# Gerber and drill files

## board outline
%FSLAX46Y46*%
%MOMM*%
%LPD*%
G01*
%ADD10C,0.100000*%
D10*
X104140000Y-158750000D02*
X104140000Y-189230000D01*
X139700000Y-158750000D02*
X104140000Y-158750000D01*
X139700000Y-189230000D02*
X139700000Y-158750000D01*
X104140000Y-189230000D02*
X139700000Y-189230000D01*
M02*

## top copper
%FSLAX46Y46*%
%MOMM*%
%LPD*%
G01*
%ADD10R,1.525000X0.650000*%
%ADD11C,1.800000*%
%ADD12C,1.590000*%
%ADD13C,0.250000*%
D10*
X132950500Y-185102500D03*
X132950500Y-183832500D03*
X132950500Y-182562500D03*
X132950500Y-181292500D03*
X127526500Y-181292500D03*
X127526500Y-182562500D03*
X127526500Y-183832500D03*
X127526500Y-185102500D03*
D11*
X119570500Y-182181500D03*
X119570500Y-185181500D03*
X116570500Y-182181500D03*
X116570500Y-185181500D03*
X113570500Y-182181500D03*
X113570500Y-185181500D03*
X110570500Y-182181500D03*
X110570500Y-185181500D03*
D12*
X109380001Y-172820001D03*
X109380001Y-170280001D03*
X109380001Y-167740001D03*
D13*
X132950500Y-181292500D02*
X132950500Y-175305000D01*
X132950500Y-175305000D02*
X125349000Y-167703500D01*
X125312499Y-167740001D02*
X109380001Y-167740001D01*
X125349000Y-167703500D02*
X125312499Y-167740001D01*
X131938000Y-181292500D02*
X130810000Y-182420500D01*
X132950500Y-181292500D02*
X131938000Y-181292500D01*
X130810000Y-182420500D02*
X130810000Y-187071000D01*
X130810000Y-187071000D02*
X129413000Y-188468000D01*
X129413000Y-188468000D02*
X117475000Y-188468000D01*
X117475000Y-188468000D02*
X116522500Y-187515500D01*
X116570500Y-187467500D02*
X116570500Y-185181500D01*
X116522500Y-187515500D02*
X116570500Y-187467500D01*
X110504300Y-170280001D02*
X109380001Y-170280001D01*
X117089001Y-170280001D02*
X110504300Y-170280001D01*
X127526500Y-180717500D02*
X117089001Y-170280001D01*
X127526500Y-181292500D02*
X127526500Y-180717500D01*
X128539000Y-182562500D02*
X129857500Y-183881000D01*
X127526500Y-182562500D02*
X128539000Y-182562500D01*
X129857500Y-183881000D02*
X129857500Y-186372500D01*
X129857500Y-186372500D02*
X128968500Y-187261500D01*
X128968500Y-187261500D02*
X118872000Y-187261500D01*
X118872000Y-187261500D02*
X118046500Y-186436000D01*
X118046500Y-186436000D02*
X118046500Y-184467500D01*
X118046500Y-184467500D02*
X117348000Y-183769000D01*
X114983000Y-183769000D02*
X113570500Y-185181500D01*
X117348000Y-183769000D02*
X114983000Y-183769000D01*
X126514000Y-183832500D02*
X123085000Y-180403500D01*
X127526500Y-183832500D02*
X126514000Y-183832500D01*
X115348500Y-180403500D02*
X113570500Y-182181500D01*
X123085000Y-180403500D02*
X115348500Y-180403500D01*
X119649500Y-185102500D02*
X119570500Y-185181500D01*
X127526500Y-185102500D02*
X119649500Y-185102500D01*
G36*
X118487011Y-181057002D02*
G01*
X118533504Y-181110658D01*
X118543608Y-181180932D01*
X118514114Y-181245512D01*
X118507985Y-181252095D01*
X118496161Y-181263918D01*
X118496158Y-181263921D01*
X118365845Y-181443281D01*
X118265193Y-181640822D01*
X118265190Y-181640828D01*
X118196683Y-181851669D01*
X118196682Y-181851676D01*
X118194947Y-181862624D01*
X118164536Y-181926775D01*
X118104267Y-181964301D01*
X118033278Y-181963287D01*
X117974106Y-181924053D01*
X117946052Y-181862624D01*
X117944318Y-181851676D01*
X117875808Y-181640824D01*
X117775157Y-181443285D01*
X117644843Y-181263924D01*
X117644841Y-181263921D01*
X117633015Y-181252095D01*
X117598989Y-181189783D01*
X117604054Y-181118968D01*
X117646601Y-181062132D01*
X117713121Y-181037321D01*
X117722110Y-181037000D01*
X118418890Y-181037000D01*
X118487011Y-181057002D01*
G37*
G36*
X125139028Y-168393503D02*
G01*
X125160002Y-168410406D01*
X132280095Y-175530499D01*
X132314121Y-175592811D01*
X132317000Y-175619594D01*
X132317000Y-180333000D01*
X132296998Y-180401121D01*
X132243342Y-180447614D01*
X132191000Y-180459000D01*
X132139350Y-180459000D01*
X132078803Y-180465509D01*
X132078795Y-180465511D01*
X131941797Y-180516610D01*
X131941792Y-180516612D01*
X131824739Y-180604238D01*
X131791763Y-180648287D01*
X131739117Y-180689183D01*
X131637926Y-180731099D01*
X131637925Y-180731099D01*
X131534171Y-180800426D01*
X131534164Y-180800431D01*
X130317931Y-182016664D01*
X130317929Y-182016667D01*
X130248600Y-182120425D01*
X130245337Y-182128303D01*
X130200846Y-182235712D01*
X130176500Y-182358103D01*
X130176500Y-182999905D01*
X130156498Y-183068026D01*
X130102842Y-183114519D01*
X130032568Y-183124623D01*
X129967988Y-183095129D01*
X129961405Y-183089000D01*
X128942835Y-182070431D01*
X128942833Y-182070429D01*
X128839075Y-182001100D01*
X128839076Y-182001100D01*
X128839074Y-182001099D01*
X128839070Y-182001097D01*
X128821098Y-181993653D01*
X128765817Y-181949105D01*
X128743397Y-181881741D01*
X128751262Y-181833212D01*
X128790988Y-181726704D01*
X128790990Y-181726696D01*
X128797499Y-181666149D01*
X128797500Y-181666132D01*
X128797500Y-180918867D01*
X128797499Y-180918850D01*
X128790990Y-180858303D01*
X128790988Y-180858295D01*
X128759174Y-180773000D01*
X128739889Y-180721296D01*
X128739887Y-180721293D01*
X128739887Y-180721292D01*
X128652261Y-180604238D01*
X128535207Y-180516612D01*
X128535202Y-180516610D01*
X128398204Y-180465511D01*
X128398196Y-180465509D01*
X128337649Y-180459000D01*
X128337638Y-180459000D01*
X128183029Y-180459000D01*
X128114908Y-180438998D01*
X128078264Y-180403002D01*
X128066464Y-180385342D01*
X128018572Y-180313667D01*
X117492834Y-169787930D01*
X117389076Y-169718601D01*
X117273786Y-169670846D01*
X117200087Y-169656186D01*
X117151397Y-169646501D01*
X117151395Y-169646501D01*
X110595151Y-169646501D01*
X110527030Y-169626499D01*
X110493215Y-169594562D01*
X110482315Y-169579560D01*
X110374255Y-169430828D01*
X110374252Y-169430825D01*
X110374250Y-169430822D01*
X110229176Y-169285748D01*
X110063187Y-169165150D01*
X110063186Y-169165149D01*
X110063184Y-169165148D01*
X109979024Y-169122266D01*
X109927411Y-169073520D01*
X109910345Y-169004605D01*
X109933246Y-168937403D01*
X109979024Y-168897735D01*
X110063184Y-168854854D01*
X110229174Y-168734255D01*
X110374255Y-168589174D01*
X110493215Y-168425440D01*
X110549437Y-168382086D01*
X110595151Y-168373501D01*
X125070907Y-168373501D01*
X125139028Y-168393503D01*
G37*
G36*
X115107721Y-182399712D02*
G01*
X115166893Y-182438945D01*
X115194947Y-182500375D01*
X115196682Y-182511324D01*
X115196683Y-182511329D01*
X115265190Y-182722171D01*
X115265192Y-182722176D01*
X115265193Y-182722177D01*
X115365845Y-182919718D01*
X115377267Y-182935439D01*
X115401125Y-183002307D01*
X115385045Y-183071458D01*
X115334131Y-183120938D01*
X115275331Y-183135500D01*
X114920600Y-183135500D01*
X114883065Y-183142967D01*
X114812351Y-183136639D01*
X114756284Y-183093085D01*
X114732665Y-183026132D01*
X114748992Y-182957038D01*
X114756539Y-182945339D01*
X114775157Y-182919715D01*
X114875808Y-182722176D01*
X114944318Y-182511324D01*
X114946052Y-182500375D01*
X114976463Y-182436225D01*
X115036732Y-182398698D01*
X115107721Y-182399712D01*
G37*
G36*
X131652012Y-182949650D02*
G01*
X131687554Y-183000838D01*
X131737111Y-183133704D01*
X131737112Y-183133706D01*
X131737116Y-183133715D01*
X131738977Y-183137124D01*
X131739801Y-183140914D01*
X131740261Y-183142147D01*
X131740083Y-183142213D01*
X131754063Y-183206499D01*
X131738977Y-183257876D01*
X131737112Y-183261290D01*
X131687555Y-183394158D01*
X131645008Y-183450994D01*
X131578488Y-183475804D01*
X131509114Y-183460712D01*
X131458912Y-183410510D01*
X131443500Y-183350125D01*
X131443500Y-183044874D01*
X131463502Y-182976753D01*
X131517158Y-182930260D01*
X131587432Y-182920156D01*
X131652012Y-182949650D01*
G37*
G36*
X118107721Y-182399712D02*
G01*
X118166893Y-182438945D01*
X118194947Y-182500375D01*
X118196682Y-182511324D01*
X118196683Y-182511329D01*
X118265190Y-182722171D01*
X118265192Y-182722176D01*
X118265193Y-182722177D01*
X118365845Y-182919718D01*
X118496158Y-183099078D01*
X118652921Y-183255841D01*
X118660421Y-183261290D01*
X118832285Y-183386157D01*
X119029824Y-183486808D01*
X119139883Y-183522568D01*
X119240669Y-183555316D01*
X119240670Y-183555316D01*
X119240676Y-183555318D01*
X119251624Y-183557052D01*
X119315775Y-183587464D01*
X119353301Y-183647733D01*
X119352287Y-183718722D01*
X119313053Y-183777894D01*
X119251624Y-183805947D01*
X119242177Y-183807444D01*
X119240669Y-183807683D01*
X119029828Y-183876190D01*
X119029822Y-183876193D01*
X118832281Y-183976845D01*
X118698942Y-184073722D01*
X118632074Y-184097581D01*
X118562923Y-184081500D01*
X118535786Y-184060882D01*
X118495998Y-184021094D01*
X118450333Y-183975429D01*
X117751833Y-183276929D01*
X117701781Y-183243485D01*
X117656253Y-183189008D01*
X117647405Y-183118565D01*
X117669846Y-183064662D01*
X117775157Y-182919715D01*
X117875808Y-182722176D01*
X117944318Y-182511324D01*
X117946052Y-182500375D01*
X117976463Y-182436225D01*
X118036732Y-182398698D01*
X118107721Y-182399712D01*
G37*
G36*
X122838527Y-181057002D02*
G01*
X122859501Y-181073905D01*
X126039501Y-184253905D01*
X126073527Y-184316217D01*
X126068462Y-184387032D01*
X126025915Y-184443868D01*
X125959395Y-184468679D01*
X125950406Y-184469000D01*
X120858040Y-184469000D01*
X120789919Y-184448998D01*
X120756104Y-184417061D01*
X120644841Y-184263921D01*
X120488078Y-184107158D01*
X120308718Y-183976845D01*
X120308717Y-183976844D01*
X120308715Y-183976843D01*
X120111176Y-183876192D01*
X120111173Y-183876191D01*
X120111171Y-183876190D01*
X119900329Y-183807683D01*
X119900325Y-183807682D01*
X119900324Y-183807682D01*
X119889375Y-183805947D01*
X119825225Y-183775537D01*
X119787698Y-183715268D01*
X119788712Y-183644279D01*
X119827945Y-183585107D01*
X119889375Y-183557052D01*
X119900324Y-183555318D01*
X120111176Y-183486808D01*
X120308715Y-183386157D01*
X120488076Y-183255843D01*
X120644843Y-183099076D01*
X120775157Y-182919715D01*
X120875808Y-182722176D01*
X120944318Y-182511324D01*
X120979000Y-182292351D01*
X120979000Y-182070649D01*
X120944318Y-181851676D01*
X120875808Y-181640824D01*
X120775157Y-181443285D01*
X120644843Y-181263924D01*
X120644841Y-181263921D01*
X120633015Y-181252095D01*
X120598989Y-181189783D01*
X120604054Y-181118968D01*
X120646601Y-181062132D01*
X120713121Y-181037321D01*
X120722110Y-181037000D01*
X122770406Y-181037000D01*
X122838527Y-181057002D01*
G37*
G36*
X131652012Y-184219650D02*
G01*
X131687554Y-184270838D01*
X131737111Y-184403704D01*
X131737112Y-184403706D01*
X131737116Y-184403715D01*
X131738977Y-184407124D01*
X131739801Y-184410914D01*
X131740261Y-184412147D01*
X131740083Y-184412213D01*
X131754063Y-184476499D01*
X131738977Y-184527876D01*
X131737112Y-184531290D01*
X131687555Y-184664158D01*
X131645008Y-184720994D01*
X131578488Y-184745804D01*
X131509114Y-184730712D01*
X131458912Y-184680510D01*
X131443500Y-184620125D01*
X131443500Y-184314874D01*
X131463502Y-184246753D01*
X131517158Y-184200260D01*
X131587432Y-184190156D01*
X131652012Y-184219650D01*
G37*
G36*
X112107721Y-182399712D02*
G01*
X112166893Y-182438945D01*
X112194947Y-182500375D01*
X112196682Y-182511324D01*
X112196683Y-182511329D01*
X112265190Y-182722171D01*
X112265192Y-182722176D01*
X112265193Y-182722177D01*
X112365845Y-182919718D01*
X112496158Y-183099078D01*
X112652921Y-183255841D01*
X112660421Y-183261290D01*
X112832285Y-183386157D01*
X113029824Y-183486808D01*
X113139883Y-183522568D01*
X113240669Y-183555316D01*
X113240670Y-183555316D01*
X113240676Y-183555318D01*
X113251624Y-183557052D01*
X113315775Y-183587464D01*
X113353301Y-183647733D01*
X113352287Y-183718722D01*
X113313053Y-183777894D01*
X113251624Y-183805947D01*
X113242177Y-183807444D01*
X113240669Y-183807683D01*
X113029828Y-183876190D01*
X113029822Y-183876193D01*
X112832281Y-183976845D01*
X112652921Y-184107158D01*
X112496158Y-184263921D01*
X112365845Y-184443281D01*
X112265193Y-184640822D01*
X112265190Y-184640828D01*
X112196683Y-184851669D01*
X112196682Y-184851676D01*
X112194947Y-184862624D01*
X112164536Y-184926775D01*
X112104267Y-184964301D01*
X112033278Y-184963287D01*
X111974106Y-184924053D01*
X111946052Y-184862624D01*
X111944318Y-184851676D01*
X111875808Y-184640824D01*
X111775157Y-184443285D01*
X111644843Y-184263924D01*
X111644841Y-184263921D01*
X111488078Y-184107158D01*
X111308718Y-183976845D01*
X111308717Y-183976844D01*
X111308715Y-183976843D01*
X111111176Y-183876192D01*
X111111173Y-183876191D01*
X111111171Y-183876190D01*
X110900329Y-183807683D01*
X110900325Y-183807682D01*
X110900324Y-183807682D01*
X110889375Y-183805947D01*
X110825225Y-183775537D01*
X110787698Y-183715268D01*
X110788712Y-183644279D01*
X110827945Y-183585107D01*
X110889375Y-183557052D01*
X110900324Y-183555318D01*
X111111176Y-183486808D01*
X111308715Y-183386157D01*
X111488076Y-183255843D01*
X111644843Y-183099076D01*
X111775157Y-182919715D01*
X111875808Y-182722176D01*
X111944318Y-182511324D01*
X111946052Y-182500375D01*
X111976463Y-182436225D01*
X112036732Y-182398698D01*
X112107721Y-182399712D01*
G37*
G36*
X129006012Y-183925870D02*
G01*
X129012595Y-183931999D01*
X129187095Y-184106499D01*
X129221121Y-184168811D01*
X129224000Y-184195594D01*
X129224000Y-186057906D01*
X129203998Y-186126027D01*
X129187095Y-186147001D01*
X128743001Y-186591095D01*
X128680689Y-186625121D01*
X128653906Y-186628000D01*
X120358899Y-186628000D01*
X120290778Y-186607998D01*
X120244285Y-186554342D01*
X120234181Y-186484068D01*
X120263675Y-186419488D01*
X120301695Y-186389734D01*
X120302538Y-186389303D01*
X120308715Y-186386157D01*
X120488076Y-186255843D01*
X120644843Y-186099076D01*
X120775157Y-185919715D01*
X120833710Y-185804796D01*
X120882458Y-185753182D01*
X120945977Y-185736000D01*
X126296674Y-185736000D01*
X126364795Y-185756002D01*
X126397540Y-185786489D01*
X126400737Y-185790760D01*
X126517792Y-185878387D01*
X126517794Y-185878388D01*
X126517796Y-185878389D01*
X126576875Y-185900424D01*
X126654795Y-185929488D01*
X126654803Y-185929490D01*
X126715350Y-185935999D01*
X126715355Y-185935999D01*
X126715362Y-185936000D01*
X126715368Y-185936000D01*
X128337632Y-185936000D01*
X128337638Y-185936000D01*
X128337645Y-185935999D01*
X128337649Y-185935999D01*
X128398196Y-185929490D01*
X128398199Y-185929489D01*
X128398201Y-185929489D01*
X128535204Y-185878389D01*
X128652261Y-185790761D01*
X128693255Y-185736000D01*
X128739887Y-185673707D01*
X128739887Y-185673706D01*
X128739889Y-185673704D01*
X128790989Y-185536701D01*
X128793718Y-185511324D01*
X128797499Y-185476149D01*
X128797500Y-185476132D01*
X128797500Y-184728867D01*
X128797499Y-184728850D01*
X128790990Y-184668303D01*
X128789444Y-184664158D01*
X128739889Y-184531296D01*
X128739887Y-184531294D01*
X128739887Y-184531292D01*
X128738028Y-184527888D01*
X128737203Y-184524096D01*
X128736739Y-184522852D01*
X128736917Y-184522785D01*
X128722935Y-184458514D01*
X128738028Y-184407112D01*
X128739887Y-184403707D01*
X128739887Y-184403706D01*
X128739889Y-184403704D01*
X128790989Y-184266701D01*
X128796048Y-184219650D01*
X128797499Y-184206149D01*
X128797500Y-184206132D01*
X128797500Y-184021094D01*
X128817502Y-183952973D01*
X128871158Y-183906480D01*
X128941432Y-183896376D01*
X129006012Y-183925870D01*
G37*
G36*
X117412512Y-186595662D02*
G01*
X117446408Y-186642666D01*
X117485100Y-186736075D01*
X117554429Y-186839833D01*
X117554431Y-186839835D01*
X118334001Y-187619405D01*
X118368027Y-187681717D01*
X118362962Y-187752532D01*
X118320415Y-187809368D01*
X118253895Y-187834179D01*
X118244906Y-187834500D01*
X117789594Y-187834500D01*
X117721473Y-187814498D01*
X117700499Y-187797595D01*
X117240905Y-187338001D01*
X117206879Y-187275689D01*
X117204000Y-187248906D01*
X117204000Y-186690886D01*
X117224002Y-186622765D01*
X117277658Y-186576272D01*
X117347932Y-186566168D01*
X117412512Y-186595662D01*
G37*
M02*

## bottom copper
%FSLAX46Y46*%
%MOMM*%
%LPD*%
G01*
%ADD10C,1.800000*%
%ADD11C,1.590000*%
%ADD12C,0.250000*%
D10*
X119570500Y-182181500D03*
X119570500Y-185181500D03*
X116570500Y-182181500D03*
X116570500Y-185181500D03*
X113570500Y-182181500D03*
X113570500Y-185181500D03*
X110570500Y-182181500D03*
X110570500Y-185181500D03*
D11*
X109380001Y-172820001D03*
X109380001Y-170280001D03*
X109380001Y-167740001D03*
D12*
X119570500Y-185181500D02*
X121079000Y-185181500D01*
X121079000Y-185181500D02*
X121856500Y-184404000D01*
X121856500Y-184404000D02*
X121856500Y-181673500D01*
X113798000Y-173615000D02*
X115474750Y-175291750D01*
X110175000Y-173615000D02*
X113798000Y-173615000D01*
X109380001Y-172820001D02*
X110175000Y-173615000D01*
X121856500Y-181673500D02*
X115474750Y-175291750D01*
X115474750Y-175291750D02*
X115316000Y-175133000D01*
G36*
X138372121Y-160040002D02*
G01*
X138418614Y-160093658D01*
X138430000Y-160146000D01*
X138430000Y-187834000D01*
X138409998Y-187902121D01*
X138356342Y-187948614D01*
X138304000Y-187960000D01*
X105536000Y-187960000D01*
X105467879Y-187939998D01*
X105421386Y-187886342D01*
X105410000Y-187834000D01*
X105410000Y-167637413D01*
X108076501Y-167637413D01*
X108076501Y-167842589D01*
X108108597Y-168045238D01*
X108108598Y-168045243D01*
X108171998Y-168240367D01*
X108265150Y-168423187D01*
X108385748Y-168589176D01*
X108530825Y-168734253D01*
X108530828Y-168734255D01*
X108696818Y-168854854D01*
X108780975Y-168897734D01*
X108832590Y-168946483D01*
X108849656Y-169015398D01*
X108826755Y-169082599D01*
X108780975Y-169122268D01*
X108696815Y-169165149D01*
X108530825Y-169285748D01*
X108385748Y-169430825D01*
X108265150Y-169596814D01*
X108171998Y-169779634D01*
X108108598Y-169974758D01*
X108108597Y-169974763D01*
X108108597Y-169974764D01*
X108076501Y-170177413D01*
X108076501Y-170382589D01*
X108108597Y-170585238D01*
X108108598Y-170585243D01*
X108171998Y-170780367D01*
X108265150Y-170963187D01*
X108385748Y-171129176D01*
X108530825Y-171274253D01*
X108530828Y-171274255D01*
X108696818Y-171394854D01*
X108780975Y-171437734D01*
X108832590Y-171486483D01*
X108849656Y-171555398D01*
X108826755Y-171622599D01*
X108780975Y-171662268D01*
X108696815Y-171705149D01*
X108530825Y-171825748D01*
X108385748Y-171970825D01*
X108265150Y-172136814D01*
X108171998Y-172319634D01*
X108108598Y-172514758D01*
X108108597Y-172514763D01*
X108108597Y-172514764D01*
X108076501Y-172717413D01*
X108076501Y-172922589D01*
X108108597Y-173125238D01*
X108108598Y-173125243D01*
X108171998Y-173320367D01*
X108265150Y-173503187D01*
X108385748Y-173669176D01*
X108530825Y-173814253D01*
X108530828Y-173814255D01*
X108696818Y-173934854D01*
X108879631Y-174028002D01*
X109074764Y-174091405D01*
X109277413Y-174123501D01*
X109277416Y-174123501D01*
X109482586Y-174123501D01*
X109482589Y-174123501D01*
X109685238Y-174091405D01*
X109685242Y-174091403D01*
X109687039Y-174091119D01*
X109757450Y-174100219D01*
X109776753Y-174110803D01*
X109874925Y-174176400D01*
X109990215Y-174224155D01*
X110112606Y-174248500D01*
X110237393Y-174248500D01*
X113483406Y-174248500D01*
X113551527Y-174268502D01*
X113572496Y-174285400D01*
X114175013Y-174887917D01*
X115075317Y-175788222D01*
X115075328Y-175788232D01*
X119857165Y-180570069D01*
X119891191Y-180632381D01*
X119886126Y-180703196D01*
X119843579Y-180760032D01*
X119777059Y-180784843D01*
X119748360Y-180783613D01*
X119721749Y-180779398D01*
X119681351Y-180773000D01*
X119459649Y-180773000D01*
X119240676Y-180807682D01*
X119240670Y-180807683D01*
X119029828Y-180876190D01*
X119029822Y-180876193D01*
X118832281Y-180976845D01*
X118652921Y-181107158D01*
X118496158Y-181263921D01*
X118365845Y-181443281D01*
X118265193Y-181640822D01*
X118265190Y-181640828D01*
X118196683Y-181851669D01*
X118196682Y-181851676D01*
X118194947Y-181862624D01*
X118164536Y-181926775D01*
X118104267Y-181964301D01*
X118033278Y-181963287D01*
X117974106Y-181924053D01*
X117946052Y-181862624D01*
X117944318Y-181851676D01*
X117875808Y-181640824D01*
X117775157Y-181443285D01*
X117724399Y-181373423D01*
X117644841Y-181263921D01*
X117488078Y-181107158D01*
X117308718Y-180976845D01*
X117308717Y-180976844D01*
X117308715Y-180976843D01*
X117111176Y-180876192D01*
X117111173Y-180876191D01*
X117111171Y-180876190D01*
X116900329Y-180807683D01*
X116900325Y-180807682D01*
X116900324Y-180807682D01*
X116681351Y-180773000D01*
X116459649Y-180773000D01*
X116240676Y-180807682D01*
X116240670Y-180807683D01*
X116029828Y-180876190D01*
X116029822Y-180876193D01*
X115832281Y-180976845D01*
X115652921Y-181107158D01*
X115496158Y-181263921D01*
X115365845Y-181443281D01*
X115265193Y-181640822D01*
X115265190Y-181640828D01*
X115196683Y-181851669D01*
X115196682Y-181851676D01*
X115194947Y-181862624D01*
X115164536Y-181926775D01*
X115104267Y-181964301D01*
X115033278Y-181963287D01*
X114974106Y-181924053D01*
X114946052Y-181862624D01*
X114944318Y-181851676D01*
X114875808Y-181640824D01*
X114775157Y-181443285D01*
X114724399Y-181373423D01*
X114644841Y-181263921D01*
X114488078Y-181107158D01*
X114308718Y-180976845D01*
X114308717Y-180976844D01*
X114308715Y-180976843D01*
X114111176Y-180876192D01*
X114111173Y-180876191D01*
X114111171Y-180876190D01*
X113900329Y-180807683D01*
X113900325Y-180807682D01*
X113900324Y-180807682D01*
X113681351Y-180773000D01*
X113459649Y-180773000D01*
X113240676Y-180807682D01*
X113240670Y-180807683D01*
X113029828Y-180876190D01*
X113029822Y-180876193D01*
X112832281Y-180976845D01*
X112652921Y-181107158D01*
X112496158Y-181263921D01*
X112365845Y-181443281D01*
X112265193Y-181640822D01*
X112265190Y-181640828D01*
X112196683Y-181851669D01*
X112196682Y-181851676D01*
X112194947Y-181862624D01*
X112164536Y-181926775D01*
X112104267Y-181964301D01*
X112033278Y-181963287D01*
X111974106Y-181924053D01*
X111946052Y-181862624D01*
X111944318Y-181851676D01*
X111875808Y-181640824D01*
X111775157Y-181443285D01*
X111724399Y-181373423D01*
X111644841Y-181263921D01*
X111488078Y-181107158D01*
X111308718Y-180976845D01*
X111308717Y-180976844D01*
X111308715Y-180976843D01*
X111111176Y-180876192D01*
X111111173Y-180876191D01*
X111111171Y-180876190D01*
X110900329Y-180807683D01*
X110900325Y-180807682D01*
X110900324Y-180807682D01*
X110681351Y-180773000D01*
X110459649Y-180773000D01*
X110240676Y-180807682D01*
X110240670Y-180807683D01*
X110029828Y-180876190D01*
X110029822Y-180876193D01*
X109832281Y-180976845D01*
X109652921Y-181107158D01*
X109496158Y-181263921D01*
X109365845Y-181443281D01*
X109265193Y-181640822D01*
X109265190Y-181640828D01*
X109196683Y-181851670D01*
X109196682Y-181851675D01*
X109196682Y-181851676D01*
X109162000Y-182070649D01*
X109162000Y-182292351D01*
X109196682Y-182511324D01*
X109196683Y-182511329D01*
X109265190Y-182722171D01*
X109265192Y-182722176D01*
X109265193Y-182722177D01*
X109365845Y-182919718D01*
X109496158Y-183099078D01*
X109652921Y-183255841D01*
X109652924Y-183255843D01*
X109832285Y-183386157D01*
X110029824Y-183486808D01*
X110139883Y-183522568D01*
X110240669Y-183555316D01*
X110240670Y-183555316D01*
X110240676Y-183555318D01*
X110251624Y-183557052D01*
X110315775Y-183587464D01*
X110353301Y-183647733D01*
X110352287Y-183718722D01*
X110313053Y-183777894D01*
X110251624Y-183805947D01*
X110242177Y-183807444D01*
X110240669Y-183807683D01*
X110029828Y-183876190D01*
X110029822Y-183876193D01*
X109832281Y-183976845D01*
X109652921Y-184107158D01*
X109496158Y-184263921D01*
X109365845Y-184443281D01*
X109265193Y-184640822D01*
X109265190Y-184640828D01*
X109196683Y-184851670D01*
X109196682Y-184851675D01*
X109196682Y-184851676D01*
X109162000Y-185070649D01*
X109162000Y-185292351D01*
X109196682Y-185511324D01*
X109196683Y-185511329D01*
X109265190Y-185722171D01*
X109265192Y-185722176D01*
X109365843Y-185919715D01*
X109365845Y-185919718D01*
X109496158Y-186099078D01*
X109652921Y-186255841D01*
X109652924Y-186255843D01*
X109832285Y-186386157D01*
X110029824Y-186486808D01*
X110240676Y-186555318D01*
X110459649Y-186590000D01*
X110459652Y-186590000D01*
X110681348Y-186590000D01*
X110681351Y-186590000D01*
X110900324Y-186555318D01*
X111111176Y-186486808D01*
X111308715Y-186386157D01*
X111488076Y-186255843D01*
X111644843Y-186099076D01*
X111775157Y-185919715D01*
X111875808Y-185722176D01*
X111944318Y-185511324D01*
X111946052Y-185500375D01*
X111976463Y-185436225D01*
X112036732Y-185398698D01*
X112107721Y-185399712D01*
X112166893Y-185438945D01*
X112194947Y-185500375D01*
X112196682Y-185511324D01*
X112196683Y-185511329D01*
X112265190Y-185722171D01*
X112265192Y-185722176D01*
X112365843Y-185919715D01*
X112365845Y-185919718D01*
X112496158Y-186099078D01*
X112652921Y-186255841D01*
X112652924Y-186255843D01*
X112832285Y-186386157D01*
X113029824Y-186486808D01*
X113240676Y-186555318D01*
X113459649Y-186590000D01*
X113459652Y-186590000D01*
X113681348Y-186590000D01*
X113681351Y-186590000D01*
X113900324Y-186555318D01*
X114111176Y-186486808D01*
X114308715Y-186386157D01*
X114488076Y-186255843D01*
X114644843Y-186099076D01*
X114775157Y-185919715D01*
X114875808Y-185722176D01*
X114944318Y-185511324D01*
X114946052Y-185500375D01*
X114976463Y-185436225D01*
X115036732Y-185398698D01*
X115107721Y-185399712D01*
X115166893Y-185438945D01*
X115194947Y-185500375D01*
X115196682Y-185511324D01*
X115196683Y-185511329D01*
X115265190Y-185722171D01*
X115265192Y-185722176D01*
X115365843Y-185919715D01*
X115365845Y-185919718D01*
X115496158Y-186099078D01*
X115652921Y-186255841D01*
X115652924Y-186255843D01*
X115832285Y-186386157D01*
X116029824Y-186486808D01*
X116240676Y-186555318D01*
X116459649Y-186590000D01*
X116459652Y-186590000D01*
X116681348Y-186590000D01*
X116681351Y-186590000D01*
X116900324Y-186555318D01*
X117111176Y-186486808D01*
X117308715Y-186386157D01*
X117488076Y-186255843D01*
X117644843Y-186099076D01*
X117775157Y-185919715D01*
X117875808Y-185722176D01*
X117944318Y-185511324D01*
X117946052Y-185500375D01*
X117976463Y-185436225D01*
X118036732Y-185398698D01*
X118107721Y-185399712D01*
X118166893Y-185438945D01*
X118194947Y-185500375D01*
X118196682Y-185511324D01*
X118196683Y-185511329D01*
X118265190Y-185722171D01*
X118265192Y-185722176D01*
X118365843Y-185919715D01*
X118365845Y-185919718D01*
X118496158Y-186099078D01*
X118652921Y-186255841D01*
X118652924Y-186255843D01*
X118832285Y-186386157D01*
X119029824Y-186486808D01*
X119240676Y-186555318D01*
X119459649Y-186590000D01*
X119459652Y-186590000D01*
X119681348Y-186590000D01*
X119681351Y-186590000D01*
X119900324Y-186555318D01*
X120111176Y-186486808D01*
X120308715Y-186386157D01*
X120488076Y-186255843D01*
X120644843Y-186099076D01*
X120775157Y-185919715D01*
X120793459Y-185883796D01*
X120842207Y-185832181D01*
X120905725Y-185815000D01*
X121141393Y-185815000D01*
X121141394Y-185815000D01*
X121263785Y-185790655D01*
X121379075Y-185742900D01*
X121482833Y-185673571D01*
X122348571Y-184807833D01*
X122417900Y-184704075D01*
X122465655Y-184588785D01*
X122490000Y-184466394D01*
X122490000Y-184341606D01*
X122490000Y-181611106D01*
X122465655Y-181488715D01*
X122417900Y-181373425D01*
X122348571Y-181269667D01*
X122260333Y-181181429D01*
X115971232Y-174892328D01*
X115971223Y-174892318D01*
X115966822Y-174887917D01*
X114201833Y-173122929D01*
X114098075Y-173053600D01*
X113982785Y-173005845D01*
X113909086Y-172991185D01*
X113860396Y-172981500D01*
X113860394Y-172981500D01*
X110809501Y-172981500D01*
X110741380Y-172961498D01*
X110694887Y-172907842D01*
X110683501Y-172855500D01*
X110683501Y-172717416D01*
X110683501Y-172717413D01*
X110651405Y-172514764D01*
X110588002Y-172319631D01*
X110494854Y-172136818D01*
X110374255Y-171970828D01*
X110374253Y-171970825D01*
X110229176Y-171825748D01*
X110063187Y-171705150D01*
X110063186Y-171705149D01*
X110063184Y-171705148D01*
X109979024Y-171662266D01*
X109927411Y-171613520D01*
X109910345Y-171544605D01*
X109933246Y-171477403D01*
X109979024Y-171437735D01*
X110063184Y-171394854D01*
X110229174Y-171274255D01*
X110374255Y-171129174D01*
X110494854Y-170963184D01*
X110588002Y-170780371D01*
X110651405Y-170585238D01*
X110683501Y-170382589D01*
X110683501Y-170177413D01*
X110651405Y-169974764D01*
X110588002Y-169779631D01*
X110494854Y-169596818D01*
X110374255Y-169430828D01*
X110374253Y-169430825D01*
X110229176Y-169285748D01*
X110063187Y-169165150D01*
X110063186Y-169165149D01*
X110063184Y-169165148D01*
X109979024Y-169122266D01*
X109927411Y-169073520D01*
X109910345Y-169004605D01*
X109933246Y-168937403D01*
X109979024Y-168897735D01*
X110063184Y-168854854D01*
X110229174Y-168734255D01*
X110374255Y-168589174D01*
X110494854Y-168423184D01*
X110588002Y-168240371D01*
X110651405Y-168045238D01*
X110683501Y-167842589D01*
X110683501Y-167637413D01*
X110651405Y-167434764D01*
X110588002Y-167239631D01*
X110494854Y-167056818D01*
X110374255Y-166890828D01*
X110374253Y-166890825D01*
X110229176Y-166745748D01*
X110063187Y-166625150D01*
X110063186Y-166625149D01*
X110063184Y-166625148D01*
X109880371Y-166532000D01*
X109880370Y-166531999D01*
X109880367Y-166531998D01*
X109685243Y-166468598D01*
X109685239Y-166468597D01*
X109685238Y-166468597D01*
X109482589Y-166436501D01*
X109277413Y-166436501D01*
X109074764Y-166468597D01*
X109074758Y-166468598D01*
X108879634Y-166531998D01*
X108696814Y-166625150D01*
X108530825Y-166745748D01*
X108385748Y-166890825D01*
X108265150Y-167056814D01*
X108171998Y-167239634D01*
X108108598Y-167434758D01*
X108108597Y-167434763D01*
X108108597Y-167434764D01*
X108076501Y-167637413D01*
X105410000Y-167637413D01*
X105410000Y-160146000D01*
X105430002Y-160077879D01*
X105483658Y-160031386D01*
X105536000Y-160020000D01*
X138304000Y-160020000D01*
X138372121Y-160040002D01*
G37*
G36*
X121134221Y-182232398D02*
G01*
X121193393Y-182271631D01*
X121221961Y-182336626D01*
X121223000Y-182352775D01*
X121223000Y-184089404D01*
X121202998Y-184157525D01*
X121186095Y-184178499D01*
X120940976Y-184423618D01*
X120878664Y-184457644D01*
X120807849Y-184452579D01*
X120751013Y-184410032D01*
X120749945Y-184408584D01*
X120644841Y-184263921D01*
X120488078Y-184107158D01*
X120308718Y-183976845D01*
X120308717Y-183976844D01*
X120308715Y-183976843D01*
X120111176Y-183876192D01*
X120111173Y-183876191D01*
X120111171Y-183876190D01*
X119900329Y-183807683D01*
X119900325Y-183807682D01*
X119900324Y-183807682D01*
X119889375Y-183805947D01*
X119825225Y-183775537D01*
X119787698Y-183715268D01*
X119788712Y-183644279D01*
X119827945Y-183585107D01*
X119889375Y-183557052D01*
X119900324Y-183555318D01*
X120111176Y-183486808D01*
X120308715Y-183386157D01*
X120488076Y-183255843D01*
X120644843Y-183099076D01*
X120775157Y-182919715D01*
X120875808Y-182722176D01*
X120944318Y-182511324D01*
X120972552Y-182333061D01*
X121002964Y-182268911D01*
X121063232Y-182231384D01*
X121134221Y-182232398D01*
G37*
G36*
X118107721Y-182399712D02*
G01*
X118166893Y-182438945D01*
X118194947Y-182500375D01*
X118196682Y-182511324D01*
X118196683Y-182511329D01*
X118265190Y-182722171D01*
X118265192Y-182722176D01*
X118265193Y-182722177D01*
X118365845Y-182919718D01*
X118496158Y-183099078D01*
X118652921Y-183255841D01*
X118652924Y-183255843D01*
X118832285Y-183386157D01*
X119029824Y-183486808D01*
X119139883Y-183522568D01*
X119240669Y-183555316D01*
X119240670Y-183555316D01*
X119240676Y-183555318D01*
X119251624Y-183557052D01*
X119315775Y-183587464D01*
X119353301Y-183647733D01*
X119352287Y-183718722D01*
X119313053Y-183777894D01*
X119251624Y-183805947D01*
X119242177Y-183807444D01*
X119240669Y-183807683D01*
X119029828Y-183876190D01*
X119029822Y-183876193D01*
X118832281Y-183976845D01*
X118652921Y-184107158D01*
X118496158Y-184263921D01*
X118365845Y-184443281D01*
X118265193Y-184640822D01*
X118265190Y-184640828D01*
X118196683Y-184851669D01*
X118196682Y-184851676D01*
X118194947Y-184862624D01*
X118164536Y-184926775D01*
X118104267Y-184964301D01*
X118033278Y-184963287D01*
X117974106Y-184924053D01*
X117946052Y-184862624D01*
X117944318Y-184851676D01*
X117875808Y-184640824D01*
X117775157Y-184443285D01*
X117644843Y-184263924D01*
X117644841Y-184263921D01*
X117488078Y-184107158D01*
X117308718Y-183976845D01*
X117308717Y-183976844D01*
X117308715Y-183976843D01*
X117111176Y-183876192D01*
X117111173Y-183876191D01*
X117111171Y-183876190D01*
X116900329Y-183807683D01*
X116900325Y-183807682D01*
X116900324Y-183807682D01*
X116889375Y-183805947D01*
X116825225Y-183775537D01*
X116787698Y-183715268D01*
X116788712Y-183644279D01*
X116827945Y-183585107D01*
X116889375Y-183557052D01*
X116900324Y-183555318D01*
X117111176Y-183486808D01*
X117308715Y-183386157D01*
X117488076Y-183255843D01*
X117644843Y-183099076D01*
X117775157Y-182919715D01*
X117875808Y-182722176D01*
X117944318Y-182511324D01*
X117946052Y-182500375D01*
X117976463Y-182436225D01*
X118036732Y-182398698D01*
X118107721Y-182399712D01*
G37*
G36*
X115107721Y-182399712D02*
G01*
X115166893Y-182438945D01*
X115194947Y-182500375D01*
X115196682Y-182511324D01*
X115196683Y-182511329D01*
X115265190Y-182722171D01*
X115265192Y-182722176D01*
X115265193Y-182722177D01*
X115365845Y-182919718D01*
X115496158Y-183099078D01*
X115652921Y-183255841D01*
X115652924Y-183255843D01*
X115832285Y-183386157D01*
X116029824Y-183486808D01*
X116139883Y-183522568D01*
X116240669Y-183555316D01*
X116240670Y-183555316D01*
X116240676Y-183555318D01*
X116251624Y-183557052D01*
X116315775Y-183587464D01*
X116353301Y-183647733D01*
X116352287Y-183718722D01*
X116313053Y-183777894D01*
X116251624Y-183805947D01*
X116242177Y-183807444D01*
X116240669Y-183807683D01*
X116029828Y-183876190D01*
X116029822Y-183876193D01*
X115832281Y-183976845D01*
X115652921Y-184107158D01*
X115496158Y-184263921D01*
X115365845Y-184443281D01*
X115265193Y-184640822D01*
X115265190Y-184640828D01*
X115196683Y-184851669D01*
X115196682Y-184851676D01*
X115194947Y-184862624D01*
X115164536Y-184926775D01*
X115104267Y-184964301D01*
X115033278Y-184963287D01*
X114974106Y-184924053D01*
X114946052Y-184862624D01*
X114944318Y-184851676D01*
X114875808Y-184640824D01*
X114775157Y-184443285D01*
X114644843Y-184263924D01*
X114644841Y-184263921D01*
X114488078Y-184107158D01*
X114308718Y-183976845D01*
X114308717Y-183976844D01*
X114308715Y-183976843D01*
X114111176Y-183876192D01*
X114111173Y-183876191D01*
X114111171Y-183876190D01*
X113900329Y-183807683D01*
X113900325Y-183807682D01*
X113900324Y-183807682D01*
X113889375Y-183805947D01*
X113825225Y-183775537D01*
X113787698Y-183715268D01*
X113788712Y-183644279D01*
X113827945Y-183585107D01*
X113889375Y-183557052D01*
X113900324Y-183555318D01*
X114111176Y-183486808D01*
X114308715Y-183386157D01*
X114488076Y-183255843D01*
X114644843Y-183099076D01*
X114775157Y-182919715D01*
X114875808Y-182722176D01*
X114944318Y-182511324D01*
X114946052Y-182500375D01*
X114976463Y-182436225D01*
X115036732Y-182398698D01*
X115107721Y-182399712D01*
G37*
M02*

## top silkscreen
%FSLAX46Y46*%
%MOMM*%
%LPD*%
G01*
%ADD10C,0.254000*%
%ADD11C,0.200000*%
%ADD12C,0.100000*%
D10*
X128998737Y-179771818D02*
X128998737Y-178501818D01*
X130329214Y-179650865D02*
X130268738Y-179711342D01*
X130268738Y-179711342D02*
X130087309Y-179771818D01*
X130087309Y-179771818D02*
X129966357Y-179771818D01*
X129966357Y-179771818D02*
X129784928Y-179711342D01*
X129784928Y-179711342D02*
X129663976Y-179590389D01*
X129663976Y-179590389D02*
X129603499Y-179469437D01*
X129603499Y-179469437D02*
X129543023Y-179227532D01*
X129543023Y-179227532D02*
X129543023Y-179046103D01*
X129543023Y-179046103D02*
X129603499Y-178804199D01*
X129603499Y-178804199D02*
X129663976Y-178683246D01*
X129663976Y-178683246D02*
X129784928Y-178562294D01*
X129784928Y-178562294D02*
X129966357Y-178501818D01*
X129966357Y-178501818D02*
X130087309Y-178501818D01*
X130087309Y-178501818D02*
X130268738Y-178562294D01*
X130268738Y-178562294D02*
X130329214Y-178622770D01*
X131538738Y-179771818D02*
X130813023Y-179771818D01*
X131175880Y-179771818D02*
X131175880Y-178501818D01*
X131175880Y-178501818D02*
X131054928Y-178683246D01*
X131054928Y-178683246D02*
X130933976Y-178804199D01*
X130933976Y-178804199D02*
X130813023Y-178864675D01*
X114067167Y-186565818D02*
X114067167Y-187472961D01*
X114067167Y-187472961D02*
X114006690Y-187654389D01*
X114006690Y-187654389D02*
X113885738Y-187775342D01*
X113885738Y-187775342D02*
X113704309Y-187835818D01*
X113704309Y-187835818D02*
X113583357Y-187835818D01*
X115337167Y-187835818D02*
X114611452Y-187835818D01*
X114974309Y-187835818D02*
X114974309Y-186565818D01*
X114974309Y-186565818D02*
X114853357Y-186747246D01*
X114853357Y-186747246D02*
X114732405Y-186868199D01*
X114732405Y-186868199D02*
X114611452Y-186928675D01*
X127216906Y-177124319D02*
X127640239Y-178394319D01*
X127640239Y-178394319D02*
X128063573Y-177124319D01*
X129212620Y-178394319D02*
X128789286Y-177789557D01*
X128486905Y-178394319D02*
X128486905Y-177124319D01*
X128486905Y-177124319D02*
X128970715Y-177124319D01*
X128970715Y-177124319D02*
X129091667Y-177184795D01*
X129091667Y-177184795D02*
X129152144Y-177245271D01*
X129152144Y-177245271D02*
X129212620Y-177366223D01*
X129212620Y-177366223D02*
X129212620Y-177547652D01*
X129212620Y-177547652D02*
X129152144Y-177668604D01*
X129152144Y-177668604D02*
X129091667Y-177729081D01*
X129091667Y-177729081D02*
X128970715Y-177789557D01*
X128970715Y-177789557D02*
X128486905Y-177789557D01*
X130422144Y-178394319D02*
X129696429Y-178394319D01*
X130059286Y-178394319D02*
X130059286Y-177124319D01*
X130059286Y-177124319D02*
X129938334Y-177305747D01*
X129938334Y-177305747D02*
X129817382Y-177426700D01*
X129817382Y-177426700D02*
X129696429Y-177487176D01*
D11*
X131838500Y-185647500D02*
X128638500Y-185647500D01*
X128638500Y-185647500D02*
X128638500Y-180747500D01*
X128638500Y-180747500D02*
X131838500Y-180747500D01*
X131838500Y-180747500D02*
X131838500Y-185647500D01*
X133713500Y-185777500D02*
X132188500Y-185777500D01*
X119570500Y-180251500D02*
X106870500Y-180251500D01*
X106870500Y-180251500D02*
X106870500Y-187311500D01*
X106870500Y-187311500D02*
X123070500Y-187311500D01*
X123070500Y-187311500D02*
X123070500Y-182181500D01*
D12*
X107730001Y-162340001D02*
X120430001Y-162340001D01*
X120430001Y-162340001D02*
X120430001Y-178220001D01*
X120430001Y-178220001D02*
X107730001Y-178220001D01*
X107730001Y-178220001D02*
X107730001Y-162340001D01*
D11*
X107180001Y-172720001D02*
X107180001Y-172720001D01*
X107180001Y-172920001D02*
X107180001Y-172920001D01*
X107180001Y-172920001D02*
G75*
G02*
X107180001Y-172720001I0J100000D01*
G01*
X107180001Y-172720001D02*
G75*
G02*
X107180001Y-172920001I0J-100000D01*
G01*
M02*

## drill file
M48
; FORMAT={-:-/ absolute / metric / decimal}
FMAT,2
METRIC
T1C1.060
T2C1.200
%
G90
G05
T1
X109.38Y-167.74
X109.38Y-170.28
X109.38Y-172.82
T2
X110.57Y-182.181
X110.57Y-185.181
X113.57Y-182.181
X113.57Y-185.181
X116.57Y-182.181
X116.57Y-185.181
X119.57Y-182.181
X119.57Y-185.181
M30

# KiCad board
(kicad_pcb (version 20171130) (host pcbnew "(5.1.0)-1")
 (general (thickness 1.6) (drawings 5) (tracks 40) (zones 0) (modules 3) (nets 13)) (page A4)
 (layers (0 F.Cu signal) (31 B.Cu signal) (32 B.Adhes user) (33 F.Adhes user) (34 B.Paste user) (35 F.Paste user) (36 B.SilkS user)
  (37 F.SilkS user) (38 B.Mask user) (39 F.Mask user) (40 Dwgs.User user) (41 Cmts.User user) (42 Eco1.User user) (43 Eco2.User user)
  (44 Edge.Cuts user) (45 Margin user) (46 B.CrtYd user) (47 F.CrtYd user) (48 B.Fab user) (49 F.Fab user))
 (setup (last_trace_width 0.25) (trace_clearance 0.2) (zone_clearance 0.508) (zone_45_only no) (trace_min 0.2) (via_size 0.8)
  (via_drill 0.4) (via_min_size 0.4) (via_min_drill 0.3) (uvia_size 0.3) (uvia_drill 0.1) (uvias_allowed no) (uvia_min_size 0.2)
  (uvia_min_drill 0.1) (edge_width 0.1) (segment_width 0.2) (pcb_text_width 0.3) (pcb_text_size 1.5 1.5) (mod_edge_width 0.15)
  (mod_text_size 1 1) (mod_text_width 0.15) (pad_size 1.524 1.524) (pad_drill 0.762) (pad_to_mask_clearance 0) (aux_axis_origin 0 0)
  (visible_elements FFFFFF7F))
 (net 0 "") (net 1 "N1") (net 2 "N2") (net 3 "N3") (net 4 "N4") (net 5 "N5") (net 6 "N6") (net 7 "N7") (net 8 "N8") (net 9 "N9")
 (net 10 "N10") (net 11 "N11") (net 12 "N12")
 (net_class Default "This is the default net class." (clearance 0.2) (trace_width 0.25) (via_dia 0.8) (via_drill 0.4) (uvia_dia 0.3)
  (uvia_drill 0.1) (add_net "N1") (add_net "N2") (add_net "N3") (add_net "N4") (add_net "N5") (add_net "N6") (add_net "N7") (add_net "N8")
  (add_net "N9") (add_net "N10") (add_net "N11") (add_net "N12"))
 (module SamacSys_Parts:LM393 (layer F.Cu) (at 130.2385 183.1975 180)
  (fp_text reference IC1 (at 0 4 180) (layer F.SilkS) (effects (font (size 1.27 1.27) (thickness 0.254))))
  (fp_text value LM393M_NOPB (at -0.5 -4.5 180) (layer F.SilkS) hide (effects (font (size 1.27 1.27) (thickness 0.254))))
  (fp_line (start -1.6 -2.45) (end 1.6 -2.45) (layer F.SilkS) (width 0.2))
  (fp_line (start 1.6 -2.45) (end 1.6 2.45) (layer F.SilkS) (width 0.2))
  (fp_line (start 1.6 2.45) (end -1.6 2.45) (layer F.SilkS) (width 0.2))
  (fp_line (start -1.6 2.45) (end -1.6 -2.45) (layer F.SilkS) (width 0.2))
  (fp_line (start -3.475 -2.58) (end -1.95 -2.58) (layer F.SilkS) (width 0.2))
  (pad 1 smd rect (at -2.712 -1.905 270) (size 0.65 1.525) (layers F.Cu F.Paste F.Mask) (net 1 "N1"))
  (pad 2 smd rect (at -2.712 -0.635 270) (size 0.65 1.525) (layers F.Cu F.Paste F.Mask) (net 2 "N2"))
  (pad 3 smd rect (at -2.712 0.635 270) (size 0.65 1.525) (layers F.Cu F.Paste F.Mask) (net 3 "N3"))
  (pad 4 smd rect (at -2.712 1.905 270) (size 0.65 1.525) (layers F.Cu F.Paste F.Mask) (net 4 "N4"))
  (pad 5 smd rect (at 2.712 1.905 270) (size 0.65 1.525) (layers F.Cu F.Paste F.Mask) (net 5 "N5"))
  (pad 6 smd rect (at 2.712 0.635 270) (size 0.65 1.525) (layers F.Cu F.Paste F.Mask) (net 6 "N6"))
  (pad 7 smd rect (at 2.712 -0.635 270) (size 0.65 1.525) (layers F.Cu F.Paste F.Mask) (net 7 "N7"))
  (pad 8 smd rect (at 2.712 -1.905 270) (size 0.65 1.525) (layers F.Cu F.Paste F.Mask) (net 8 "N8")))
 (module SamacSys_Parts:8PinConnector (layer F.Cu) (at 119.5705 182.1815)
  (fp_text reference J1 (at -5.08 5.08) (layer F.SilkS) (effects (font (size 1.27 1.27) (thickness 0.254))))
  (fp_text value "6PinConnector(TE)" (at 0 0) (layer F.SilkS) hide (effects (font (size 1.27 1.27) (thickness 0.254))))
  (fp_line (start 0 -1.93) (end -12.7 -1.93) (layer F.SilkS) (width 0.2))
  (fp_line (start -12.7 -1.93) (end -12.7 5.13) (layer F.SilkS) (width 0.2))
  (fp_line (start -12.7 5.13) (end 3.5 5.13) (layer F.SilkS) (width 0.2))
  (fp_line (start 3.5 5.13) (end 3.5 0) (layer F.SilkS) (width 0.2))
  (pad 1 thru_hole circle (at 0 0) (size 1.8 1.8) (drill 1.2) (layers *.Cu *.Mask) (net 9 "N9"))
  (pad 2 thru_hole circle (at 0 3) (size 1.8 1.8) (drill 1.2) (layers *.Cu *.Mask) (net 8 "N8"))
  (pad 3 thru_hole circle (at -3 0) (size 1.8 1.8) (drill 1.2) (layers *.Cu *.Mask) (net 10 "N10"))
  (pad 4 thru_hole circle (at -3 3) (size 1.8 1.8) (drill 1.2) (layers *.Cu *.Mask) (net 4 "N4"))
  (pad 5 thru_hole circle (at -6 0) (size 1.8 1.8) (drill 1.2) (layers *.Cu *.Mask) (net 7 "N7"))
  (pad 6 thru_hole circle (at -6 3) (size 1.8 1.8) (drill 1.2) (layers *.Cu *.Mask) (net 6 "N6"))
  (pad 7 thru_hole circle (at -9 0) (size 1.8 1.8) (drill 1.2) (layers *.Cu *.Mask) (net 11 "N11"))
  (pad 8 thru_hole circle (at -9 3) (size 1.8 1.8) (drill 1.2) (layers *.Cu *.Mask) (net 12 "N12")))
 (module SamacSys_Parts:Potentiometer (layer F.Cu) (at 109.380001 172.820001)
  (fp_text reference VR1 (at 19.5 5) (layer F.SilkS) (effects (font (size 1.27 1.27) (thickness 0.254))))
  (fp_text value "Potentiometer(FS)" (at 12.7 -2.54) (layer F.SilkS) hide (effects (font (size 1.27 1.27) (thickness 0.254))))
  (fp_line (start -1.65 -10.48) (end 11.05 -10.48) (layer F.SilkS) (width 0.1))
  (fp_line (start 11.05 -10.48) (end 11.05 5.4) (layer F.SilkS) (width 0.1))
  (fp_line (start 11.05 5.4) (end -1.65 5.4) (layer F.SilkS) (width 0.1))
  (fp_line (start -1.65 5.4) (end -1.65 -10.48) (layer F.SilkS) (width 0.1))
  (fp_line (start -2.2 -0.1) (end -2.2 -0.1) (layer F.SilkS) (width 0.2))
  (fp_line (start -2.2 0.1) (end -2.2 0.1) (layer F.SilkS) (width 0.2))
  (fp_arc (start -2.2 0) (end -2.2 -0.1) (angle -180) (layer F.SilkS) (width 0.2))
  (fp_arc (start -2.2 0) (end -2.2 0.1) (angle -180) (layer F.SilkS) (width 0.2))
  (pad 1 thru_hole circle (at 0 0) (size 1.59 1.59) (drill 1.06) (layers *.Cu *.Mask) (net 8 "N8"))
  (pad 2 thru_hole circle (at 0 -2.54) (size 1.59 1.59) (drill 1.06) (layers *.Cu *.Mask) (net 5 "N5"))
  (pad 3 thru_hole circle (at 0 -5.08) (size 1.59 1.59) (drill 1.06) (layers *.Cu *.Mask) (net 4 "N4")))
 (gr_line (start 104.14 158.75) (end 104.14 189.23) (layer Edge.Cuts) (width 0.1))
 (gr_line (start 139.7 158.75) (end 104.14 158.75) (layer Edge.Cuts) (width 0.1))
 (gr_line (start 139.7 189.23) (end 139.7 158.75) (layer Edge.Cuts) (width 0.1))
 (gr_line (start 104.14 189.23) (end 139.7 189.23) (layer Edge.Cuts) (width 0.1))
 (segment (start 132.9505 181.2925) (end 132.9505 175.305) (width 0.25) (layer F.Cu) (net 4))
 (segment (start 132.9505 175.305) (end 125.349 167.7035) (width 0.25) (layer F.Cu) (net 4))
 (segment (start 125.312499 167.740001) (end 109.380001 167.740001) (width 0.25) (layer F.Cu) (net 4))
 (segment (start 125.349 167.7035) (end 125.312499 167.740001) (width 0.25) (layer F.Cu) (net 4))
 (segment (start 131.938 181.2925) (end 130.81 182.4205) (width 0.25) (layer F.Cu) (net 4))
 (segment (start 132.9505 181.2925) (end 131.938 181.2925) (width 0.25) (layer F.Cu) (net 4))
 (segment (start 130.81 182.4205) (end 130.81 187.071) (width 0.25) (layer F.Cu) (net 4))
 (segment (start 130.81 187.071) (end 129.413 188.468) (width 0.25) (layer F.Cu) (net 4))
 (segment (start 129.413 188.468) (end 117.475 188.468) (width 0.25) (layer F.Cu) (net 4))
 (segment (start 117.475 188.468) (end 116.5225 187.5155) (width 0.25) (layer F.Cu) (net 4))
 (segment (start 116.5705 187.4675) (end 116.5705 185.1815) (width 0.25) (layer F.Cu) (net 4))
 (segment (start 116.5225 187.5155) (end 116.5705 187.4675) (width 0.25) (layer F.Cu) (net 4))
 (segment (start 110.5043 170.280001) (end 109.380001 170.280001) (width 0.25) (layer F.Cu) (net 5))
 (segment (start 117.089001 170.280001) (end 110.5043 170.280001) (width 0.25) (layer F.Cu) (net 5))
 (segment (start 127.5265 180.7175) (end 117.089001 170.280001) (width 0.25) (layer F.Cu) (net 5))
 (segment (start 127.5265 181.2925) (end 127.5265 180.7175) (width 0.25) (layer F.Cu) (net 5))
 (segment (start 128.539 182.5625) (end 129.8575 183.881) (width 0.25) (layer F.Cu) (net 6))
 (segment (start 127.5265 182.5625) (end 128.539 182.5625) (width 0.25) (layer F.Cu) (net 6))
 (segment (start 129.8575 183.881) (end 129.8575 186.3725) (width 0.25) (layer F.Cu) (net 6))
 (segment (start 129.8575 186.3725) (end 128.9685 187.2615) (width 0.25) (layer F.Cu) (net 6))
 (segment (start 128.9685 187.2615) (end 118.872 187.2615) (width 0.25) (layer F.Cu) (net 6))
 (segment (start 118.872 187.2615) (end 118.0465 186.436) (width 0.25) (layer F.Cu) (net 6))
 (segment (start 118.0465 186.436) (end 118.0465 184.4675) (width 0.25) (layer F.Cu) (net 6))
 (segment (start 118.0465 184.4675) (end 117.348 183.769) (width 0.25) (layer F.Cu) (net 6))
 (segment (start 114.983 183.769) (end 113.5705 185.1815) (width 0.25) (layer F.Cu) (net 6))
 (segment (start 117.348 183.769) (end 114.983 183.769) (width 0.25) (layer F.Cu) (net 6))
 (segment (start 126.514 183.8325) (end 123.085 180.4035) (width 0.25) (layer F.Cu) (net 7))
 (segment (start 127.5265 183.8325) (end 126.514 183.8325) (width 0.25) (layer F.Cu) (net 7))
 (segment (start 115.3485 180.4035) (end 113.5705 182.1815) (width 0.25) (layer F.Cu) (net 7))
 (segment (start 123.085 180.4035) (end 115.3485 180.4035) (width 0.25) (layer F.Cu) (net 7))
 (segment (start 119.6495 185.1025) (end 119.5705 185.1815) (width 0.25) (layer F.Cu) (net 8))
 (segment (start 127.5265 185.1025) (end 119.6495 185.1025) (width 0.25) (layer F.Cu) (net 8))
 (segment (start 119.5705 185.1815) (end 121.079 185.1815) (width 0.25) (layer B.Cu) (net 8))
 (segment (start 121.079 185.1815) (end 121.8565 184.404) (width 0.25) (layer B.Cu) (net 8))
 (segment (start 121.8565 184.404) (end 121.8565 181.6735) (width 0.25) (layer B.Cu) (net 8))
 (segment (start 113.798 173.615) (end 115.47475 175.29175) (width 0.25) (layer B.Cu) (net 8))
 (segment (start 110.175 173.615) (end 113.798 173.615) (width 0.25) (layer B.Cu) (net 8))
 (segment (start 109.380001 172.820001) (end 110.175 173.615) (width 0.25) (layer B.Cu) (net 8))
 (segment (start 121.8565 181.6735) (end 115.47475 175.29175) (width 0.25) (layer B.Cu) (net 8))
 (segment (start 115.47475 175.29175) (end 115.316 175.133) (width 0.25) (layer B.Cu) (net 8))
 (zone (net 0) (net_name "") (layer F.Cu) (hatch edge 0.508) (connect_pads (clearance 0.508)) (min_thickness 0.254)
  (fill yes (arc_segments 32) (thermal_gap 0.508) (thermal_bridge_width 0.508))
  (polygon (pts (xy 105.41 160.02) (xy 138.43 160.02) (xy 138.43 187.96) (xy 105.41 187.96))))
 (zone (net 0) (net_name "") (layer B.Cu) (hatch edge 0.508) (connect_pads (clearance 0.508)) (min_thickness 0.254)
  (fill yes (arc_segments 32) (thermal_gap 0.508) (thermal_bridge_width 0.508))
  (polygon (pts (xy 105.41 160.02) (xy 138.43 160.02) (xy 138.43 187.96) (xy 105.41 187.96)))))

